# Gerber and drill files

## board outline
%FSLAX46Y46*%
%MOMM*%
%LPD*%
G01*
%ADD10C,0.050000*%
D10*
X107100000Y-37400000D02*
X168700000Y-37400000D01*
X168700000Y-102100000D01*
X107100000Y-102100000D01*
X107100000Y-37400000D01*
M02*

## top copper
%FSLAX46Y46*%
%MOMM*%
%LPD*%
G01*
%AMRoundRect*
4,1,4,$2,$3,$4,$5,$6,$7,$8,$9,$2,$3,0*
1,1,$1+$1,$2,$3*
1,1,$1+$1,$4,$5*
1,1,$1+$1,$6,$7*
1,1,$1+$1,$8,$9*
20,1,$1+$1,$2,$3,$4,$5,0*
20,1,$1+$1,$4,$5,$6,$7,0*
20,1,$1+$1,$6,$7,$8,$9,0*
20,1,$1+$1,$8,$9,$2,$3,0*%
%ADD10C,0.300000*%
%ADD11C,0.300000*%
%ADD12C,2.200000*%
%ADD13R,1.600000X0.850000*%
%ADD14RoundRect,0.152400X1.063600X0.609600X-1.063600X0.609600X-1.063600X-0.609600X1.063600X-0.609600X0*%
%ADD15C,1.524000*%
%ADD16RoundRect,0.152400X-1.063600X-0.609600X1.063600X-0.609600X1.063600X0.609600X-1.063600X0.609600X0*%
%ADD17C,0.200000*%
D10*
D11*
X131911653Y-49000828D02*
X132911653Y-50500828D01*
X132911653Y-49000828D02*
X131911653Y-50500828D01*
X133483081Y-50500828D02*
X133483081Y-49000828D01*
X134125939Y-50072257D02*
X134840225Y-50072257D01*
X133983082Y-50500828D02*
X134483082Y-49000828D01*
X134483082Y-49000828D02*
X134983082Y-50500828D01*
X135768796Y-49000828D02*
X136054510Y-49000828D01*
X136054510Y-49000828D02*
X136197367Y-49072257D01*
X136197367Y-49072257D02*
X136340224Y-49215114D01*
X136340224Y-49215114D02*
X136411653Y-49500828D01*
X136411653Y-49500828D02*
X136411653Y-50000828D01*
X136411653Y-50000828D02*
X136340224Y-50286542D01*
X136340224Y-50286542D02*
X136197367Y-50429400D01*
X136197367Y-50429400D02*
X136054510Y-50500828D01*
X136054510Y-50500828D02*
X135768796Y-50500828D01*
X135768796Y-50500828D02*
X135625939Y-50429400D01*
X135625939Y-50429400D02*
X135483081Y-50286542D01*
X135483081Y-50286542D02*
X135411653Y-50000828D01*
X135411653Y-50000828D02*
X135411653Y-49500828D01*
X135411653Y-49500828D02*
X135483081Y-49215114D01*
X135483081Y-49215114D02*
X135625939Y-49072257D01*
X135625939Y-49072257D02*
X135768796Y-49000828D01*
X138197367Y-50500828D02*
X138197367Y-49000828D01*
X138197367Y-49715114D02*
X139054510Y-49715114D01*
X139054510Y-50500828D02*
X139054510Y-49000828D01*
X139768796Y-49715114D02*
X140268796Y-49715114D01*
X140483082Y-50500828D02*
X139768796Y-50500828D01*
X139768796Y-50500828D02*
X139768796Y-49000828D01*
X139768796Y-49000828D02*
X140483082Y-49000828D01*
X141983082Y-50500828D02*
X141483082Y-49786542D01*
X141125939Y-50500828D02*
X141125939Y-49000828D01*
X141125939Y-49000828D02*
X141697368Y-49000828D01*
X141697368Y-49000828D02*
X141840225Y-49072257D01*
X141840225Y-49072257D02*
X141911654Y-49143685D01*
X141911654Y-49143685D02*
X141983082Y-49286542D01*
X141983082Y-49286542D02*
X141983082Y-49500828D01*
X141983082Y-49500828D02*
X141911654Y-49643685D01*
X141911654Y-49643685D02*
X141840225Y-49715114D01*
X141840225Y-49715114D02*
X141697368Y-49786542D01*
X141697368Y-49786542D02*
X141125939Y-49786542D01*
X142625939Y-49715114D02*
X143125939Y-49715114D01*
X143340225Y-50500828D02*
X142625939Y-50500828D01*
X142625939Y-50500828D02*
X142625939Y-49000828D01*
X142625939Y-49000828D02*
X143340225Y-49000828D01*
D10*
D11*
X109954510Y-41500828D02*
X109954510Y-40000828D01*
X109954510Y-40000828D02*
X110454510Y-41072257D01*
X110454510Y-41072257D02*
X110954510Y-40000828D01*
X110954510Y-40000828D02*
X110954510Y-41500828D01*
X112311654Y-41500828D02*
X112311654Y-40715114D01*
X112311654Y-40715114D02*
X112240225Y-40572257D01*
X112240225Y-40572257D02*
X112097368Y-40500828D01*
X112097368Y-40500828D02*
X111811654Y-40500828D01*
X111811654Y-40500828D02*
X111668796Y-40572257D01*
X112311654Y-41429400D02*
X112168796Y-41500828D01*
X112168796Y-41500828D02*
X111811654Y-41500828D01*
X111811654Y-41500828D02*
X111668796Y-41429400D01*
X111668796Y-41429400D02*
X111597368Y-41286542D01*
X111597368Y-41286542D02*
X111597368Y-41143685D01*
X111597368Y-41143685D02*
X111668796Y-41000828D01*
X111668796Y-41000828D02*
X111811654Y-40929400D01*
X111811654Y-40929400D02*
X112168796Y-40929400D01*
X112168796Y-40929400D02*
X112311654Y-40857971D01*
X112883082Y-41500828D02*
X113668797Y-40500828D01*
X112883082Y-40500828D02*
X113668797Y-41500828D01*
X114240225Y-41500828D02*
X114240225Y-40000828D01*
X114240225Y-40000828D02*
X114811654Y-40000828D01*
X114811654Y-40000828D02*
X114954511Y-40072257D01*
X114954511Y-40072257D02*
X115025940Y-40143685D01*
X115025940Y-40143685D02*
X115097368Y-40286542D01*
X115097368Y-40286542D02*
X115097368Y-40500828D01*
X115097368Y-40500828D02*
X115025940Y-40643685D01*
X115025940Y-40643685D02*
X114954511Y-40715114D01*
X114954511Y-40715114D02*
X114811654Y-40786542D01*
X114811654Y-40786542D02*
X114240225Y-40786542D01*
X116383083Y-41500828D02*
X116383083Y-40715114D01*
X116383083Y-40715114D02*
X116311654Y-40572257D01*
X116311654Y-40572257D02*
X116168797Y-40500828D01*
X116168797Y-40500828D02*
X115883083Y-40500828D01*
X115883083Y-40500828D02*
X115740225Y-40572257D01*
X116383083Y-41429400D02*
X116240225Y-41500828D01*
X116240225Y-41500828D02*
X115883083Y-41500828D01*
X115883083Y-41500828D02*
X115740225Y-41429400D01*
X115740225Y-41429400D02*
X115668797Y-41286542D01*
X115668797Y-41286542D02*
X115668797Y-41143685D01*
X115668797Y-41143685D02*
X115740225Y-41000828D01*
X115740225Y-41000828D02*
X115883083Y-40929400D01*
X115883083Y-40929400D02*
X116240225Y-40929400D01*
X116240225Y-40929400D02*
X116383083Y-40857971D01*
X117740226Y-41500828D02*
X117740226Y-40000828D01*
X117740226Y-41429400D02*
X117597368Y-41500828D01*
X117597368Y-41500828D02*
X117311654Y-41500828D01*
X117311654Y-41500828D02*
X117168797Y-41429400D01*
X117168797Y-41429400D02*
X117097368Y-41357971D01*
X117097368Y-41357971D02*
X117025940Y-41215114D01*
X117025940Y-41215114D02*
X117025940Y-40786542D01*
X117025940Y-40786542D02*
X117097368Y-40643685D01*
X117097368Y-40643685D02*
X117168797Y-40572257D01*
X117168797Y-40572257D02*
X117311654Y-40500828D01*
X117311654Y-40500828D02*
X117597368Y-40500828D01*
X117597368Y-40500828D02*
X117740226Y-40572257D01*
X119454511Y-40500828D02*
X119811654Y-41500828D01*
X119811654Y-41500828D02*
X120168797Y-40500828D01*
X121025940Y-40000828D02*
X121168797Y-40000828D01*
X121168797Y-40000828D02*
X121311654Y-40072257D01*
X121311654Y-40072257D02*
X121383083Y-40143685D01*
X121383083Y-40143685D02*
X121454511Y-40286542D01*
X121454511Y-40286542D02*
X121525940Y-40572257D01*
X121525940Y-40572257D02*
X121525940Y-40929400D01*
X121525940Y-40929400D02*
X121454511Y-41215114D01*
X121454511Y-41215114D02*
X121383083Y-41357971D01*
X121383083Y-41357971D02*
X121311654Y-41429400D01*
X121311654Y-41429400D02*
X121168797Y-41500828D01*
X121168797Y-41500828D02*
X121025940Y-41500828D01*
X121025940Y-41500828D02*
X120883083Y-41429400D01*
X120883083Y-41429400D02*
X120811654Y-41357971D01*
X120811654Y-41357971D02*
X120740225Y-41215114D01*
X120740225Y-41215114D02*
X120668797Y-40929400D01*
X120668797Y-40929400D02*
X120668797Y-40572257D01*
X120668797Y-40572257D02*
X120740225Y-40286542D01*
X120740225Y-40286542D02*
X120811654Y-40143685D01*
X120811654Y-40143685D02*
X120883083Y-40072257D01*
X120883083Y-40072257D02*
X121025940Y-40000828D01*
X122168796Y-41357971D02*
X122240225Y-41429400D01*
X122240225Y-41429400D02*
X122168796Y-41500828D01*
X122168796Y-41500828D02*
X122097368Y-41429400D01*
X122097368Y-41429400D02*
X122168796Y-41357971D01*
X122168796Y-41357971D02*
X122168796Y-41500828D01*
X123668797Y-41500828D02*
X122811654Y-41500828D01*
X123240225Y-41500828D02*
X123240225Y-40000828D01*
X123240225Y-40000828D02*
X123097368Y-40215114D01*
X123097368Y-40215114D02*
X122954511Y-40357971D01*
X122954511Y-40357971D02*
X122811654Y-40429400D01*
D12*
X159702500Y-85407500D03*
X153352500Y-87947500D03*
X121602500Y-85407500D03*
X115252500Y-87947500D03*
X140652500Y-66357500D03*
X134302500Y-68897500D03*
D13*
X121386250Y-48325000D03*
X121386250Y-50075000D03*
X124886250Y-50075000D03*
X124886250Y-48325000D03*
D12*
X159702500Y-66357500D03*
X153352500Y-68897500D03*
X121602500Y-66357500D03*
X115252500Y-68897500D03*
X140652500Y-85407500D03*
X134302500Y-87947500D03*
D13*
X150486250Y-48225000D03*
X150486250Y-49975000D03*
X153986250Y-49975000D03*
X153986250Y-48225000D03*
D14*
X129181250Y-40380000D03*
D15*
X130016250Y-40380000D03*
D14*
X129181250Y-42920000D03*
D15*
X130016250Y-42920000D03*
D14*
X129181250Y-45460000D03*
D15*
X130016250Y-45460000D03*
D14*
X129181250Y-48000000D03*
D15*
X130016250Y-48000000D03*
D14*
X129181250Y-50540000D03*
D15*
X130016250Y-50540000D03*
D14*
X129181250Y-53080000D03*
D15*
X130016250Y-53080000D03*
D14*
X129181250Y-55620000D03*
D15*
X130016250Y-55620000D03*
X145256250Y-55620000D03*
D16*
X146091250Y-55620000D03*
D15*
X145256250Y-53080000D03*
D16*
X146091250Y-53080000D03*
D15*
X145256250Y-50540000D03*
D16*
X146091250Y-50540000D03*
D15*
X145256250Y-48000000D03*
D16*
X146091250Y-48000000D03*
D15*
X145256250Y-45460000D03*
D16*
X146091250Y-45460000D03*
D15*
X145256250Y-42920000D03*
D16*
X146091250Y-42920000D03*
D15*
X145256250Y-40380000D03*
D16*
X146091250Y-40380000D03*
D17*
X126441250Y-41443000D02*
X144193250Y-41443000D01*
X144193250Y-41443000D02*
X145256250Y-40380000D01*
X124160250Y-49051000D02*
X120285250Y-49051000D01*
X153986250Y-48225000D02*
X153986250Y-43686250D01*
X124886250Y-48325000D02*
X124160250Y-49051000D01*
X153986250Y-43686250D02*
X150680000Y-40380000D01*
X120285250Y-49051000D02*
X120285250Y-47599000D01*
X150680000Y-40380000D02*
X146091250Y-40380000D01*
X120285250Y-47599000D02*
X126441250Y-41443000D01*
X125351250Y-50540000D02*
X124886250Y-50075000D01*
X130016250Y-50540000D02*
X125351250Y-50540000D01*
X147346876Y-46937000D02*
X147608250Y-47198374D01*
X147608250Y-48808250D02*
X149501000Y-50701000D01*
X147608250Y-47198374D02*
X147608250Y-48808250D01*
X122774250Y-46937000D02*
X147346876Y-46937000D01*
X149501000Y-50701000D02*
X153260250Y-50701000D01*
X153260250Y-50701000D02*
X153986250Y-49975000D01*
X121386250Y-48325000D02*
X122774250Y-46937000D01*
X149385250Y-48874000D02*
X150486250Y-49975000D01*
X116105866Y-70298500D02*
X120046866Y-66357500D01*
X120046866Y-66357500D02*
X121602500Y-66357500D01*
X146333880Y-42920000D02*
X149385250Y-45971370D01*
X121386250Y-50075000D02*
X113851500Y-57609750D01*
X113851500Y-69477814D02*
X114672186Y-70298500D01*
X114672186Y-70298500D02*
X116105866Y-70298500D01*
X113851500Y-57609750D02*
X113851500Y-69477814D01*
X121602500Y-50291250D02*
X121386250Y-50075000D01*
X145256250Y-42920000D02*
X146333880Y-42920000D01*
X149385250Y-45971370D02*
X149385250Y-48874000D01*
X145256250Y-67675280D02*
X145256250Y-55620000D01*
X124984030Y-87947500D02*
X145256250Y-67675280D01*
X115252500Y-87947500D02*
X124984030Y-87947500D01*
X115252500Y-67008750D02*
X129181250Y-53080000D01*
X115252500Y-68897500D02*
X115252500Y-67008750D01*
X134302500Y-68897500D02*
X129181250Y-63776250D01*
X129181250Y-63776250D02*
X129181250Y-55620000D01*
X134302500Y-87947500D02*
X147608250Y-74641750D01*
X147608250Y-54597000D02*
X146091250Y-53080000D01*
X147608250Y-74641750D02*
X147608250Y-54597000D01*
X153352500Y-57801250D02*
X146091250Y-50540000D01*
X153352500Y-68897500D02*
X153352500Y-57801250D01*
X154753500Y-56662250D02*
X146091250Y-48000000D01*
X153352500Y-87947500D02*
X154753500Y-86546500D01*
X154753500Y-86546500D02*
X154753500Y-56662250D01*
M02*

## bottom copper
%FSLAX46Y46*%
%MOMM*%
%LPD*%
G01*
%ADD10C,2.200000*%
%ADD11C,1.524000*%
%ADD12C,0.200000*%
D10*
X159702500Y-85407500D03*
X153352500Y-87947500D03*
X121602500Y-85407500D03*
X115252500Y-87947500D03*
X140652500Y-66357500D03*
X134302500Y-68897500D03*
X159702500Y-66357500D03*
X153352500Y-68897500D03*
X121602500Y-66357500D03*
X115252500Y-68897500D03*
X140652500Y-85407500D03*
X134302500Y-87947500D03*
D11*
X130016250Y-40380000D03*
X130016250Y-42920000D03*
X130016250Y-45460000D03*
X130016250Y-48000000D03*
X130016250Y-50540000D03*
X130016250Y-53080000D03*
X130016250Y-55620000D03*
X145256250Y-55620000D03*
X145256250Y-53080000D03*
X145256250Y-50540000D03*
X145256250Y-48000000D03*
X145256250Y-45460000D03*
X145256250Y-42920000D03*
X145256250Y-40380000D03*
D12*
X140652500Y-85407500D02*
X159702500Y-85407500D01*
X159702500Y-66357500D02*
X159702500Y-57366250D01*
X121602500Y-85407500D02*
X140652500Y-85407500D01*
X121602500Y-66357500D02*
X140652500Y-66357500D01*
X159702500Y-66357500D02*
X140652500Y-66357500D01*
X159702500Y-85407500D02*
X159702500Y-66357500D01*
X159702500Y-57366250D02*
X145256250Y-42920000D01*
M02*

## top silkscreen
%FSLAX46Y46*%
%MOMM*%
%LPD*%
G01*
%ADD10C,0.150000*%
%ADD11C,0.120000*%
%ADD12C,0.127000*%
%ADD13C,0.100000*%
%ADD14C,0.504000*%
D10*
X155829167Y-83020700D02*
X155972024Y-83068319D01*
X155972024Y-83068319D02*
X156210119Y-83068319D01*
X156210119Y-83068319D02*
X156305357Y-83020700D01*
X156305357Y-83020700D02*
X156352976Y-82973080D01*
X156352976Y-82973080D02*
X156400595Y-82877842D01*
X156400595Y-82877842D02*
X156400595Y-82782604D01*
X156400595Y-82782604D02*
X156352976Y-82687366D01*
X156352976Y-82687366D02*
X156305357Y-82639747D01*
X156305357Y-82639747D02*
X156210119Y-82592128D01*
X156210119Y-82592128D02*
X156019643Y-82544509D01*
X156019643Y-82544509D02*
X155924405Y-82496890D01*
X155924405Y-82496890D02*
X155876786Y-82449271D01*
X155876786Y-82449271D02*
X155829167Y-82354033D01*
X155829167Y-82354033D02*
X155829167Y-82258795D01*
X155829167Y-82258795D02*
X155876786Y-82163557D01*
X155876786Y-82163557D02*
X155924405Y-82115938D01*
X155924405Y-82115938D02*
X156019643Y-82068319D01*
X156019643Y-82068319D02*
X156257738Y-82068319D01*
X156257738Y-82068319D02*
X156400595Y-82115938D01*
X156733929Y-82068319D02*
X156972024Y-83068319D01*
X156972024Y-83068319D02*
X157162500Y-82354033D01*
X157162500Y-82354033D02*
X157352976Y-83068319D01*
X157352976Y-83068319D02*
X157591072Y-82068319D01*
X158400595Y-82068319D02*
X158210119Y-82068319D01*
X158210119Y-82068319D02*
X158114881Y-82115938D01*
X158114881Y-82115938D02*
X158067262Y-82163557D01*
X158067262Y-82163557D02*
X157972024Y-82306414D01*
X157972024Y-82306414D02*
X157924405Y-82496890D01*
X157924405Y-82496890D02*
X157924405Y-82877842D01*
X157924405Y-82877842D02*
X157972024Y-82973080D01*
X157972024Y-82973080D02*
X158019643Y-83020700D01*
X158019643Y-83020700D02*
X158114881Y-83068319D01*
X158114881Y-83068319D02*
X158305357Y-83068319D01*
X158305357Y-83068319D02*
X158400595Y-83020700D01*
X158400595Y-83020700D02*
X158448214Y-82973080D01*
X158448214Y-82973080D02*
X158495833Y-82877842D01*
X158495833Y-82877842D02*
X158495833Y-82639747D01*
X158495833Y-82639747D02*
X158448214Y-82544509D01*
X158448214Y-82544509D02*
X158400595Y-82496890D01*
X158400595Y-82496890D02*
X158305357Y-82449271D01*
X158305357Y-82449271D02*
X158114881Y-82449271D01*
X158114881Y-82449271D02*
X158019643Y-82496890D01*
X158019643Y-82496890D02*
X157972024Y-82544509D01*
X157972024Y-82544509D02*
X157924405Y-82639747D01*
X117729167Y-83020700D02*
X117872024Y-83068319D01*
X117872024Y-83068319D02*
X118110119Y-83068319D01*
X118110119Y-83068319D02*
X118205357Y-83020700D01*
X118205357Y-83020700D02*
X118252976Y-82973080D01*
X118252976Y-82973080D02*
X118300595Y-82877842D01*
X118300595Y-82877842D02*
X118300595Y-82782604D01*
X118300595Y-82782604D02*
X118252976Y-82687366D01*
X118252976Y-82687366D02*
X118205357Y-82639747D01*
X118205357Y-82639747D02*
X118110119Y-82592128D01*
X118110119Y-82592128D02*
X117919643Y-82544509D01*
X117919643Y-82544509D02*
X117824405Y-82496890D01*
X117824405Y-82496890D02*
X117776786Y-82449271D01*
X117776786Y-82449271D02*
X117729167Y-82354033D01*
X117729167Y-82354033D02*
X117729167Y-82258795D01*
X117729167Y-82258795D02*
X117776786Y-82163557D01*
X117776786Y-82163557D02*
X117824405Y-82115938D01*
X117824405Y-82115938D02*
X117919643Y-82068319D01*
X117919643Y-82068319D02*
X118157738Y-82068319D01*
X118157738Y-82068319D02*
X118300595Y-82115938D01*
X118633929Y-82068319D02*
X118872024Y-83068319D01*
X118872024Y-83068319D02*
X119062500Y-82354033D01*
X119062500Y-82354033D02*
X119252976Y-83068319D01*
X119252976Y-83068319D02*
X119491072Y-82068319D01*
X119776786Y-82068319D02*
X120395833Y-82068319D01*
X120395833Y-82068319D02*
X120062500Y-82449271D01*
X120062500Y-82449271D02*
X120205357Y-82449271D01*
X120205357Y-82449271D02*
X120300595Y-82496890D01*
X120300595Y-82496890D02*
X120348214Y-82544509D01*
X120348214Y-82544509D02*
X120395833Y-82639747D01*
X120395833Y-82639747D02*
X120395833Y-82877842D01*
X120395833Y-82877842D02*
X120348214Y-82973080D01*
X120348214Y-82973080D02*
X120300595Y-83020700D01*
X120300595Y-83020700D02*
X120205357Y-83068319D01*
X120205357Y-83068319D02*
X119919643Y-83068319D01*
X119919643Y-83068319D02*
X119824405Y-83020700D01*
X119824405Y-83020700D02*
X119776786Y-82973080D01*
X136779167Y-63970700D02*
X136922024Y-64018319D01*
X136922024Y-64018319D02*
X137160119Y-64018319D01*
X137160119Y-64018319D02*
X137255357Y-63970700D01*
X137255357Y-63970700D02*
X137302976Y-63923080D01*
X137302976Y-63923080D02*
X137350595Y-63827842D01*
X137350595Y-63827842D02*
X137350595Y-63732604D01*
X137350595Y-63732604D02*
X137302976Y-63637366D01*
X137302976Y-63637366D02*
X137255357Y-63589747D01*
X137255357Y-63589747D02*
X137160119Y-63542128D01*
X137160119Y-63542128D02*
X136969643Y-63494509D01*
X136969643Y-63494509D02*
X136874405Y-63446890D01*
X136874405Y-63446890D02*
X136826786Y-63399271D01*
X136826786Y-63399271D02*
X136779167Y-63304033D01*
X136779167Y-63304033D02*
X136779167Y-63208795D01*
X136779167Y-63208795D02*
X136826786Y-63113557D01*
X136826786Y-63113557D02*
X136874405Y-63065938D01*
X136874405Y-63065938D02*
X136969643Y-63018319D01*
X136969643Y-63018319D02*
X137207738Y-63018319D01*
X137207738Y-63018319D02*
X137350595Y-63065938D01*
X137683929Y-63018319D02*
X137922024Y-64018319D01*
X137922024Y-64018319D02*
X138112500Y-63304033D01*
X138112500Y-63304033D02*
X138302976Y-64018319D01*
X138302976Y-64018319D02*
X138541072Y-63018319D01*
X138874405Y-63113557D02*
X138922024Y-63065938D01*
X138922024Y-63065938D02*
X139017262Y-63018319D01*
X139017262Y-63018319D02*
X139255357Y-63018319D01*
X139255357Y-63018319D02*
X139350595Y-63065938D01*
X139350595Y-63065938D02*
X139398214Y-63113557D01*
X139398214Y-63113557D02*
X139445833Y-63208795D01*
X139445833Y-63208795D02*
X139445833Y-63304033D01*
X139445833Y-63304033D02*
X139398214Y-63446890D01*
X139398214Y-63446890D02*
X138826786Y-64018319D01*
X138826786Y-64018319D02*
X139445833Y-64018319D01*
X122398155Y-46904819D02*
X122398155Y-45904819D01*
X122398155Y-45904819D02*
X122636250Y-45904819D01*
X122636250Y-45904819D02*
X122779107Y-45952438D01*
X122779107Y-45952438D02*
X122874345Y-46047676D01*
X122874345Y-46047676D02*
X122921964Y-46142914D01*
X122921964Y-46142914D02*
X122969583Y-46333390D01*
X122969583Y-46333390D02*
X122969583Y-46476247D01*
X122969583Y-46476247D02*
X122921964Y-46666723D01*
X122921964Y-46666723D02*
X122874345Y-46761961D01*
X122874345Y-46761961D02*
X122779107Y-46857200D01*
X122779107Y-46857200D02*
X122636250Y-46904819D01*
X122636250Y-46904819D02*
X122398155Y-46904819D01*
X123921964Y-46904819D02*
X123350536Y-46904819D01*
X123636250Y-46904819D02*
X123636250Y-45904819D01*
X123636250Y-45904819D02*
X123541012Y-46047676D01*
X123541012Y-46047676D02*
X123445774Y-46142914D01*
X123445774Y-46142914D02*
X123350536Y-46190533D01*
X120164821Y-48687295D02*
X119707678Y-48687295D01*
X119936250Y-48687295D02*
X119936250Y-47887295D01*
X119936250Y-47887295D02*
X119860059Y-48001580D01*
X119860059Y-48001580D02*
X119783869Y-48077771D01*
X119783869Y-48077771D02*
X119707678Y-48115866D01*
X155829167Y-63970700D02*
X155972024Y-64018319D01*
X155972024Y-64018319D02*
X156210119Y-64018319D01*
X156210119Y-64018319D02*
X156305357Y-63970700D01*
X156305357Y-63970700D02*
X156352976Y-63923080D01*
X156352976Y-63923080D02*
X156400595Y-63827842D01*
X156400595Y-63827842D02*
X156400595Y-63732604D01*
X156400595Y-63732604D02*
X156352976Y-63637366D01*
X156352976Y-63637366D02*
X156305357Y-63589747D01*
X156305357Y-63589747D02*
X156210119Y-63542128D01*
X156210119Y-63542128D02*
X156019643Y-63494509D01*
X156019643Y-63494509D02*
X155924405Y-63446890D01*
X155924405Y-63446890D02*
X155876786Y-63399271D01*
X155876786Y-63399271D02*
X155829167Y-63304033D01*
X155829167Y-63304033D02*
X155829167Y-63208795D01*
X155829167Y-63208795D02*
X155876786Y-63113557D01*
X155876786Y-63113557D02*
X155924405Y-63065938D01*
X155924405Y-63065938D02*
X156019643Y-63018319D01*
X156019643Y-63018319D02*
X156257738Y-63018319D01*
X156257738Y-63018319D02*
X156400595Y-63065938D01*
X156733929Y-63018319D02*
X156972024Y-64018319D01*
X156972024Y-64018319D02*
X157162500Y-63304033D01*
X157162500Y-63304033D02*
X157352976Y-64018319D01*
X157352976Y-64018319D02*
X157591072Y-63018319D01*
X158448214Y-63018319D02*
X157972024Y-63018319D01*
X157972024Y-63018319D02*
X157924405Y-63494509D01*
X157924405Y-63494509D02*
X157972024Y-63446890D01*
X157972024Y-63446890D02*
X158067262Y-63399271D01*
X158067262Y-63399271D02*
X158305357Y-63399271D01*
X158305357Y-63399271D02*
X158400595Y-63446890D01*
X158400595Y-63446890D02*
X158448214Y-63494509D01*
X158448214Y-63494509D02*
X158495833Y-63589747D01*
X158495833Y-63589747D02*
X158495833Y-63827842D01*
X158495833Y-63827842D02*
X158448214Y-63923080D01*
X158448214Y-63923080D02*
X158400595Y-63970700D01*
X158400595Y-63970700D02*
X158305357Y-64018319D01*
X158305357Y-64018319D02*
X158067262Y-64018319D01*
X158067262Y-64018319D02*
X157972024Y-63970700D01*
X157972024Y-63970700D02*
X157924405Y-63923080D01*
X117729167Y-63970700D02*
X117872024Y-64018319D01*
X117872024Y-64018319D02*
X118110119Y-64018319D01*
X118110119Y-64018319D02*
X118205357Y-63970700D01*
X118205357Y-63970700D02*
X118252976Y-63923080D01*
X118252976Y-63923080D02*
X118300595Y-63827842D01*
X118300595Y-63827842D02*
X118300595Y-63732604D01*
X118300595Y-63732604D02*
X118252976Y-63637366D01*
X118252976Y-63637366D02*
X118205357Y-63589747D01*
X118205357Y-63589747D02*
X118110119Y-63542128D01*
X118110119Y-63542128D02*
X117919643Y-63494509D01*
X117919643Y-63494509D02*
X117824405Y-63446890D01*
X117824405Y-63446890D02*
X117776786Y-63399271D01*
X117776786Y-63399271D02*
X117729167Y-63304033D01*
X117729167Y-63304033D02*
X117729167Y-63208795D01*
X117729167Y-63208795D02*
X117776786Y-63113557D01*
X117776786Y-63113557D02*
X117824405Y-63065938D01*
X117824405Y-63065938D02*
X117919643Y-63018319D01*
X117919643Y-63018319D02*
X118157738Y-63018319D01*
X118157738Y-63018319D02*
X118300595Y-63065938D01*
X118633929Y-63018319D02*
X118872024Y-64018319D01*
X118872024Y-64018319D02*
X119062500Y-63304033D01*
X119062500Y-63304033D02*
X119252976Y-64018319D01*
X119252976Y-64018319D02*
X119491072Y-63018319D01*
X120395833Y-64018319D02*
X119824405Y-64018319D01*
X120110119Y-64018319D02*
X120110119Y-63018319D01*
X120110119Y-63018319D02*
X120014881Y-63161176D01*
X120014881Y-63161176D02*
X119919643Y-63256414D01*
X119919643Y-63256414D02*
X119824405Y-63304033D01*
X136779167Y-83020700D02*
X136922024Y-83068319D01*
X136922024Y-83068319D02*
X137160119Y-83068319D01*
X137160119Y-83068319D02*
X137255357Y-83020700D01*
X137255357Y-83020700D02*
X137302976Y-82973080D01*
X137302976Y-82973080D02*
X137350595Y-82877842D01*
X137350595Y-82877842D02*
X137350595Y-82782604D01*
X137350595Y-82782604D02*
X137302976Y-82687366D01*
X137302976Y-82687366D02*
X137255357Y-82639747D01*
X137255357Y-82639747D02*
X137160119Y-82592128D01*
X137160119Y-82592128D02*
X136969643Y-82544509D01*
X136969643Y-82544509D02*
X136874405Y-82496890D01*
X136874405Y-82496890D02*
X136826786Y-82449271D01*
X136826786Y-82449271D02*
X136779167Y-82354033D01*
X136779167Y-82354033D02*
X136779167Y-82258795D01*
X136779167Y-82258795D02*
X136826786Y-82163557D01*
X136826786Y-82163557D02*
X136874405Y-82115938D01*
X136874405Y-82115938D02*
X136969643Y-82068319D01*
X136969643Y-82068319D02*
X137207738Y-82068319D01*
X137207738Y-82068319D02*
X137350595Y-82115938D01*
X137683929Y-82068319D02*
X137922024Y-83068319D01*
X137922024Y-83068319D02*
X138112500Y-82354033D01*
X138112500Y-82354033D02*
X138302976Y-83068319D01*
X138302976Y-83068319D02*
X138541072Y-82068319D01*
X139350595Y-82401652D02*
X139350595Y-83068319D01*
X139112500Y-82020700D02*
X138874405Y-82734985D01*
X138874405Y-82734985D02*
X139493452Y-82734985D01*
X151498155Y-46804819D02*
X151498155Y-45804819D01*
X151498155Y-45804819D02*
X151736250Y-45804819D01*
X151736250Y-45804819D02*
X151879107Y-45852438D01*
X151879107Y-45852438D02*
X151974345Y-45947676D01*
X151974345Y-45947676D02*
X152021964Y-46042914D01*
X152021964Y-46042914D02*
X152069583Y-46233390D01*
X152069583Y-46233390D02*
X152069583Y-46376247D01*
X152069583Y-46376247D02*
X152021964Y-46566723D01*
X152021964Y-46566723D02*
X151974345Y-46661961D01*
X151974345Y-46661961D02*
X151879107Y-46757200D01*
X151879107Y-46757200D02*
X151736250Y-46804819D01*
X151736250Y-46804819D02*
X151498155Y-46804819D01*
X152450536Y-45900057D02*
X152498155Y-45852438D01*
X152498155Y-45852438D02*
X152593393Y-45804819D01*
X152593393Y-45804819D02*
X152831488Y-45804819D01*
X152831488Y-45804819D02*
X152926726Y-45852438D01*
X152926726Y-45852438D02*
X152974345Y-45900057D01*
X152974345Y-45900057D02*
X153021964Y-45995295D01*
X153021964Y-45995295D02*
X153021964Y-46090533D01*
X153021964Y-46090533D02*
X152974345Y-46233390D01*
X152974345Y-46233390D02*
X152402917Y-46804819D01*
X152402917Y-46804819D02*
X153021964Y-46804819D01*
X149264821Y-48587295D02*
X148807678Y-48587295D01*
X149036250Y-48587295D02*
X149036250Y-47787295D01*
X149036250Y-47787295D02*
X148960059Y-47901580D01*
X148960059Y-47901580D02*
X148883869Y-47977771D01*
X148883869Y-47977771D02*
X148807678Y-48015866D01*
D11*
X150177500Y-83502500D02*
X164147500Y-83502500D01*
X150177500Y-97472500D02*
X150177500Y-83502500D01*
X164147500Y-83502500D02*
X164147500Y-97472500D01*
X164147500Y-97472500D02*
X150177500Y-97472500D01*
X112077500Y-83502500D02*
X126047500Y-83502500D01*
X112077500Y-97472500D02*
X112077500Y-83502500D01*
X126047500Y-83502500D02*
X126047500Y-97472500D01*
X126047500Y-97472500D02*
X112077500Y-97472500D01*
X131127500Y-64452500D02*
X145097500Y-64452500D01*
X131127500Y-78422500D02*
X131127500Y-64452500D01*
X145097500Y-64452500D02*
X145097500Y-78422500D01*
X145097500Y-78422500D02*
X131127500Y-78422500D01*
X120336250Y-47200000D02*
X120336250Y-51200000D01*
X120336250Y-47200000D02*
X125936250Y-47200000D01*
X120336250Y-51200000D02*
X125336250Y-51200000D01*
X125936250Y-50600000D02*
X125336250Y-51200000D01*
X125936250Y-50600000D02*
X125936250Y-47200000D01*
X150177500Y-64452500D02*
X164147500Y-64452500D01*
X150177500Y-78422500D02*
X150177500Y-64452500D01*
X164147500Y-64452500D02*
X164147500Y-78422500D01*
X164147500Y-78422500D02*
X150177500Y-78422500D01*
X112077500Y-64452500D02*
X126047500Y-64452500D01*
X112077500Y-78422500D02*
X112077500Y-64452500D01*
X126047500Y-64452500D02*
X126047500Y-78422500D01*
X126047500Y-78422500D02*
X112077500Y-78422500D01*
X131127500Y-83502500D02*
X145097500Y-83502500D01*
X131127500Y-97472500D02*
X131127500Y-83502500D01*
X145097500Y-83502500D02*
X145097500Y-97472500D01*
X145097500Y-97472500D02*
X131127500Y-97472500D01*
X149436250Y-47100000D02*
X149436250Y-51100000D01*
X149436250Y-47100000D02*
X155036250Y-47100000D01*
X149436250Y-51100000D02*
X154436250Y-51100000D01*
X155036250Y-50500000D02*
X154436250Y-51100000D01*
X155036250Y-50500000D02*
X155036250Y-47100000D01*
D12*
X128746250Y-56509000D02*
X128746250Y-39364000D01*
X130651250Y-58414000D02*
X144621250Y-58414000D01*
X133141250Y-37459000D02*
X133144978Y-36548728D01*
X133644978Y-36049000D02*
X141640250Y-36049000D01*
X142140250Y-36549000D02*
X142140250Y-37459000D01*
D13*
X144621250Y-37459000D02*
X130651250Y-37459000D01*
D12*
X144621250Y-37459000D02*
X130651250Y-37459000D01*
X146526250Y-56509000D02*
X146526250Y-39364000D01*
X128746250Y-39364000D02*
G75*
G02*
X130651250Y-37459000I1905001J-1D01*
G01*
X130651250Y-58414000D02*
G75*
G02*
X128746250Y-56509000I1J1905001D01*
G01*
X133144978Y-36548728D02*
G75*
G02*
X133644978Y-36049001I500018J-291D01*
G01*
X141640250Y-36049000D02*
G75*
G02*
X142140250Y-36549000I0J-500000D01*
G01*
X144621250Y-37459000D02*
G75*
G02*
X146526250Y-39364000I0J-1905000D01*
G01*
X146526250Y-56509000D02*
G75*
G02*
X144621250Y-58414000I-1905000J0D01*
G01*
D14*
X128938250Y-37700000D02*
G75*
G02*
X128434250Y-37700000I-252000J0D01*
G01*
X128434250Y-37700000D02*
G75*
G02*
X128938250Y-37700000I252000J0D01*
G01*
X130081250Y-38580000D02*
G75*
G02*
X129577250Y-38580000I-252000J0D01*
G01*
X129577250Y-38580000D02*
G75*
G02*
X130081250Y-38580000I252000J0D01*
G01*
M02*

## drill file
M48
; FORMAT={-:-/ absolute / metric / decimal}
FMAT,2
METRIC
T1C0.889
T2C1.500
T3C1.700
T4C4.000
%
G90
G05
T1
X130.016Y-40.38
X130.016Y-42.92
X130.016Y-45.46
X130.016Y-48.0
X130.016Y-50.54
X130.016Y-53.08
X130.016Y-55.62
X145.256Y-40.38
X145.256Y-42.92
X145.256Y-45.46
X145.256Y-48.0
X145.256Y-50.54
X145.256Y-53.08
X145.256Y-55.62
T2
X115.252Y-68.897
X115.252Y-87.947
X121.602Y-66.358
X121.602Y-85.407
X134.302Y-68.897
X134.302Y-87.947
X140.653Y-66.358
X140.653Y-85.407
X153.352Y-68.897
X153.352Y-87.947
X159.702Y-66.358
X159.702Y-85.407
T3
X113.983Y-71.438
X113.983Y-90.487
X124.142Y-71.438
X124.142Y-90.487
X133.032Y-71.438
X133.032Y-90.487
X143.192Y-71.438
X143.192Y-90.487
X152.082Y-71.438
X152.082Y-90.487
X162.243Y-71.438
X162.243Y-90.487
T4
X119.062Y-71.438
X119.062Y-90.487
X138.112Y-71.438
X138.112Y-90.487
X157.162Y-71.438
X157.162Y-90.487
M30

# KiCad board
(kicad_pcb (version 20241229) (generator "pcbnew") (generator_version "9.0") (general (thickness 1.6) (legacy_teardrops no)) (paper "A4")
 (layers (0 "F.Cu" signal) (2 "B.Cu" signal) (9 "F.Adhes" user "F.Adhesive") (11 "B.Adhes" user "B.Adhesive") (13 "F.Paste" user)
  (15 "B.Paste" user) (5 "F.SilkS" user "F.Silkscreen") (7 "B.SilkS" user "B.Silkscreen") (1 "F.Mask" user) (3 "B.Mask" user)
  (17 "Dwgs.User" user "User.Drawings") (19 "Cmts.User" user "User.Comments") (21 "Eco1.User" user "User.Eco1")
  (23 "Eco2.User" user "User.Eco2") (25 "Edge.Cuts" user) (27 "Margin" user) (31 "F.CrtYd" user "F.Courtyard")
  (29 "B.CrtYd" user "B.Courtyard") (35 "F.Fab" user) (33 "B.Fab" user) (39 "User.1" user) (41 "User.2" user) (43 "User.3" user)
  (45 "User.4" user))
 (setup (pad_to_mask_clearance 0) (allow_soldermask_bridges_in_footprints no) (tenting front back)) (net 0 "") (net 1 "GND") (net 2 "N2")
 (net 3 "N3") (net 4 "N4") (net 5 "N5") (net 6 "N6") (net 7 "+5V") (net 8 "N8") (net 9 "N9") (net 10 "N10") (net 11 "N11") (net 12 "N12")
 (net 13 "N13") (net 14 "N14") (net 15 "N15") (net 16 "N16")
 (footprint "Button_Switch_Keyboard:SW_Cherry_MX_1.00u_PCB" (layer "F.Cu") (at 159.7025 85.4075)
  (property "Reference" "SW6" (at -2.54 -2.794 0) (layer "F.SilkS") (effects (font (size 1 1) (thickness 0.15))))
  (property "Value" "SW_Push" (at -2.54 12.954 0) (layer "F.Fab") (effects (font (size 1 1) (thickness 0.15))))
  (fp_line (start -9.525 -1.905) (end 4.445 -1.905) (stroke (width 0.12) (type solid)) (layer "F.SilkS"))
  (fp_line (start -9.525 12.065) (end -9.525 -1.905) (stroke (width 0.12) (type solid)) (layer "F.SilkS"))
  (fp_line (start 4.445 -1.905) (end 4.445 12.065) (stroke (width 0.12) (type solid)) (layer "F.SilkS"))
  (fp_line (start 4.445 12.065) (end -9.525 12.065) (stroke (width 0.12) (type solid)) (layer "F.SilkS"))
  (pad "" np_thru_hole circle (at -7.62 5.08) (size 1.7 1.7) (drill 1.7) (layers "*.Cu" "*.Mask"))
  (pad "" np_thru_hole circle (at -2.54 5.08) (size 4 4) (drill 4) (layers "*.Cu" "*.Mask"))
  (pad "" np_thru_hole circle (at 2.54 5.08) (size 1.7 1.7) (drill 1.7) (layers "*.Cu" "*.Mask"))
  (pad "1" thru_hole circle (at 0 0) (size 2.2 2.2) (drill 1.5) (layers "*.Cu" "*.Mask") (remove_unused_layers no) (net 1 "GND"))
  (pad "2" thru_hole circle (at -6.35 2.54) (size 2.2 2.2) (drill 1.5) (layers "*.Cu" "*.Mask") (remove_unused_layers no) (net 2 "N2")))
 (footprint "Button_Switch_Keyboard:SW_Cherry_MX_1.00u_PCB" (layer "F.Cu") (at 121.6025 85.4075)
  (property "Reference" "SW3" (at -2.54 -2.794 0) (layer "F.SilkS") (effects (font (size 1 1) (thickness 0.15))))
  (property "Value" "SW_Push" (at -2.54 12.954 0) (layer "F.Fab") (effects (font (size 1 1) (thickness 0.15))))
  (fp_line (start -9.525 -1.905) (end 4.445 -1.905) (stroke (width 0.12) (type solid)) (layer "F.SilkS"))
  (fp_line (start -9.525 12.065) (end -9.525 -1.905) (stroke (width 0.12) (type solid)) (layer "F.SilkS"))
  (fp_line (start 4.445 -1.905) (end 4.445 12.065) (stroke (width 0.12) (type solid)) (layer "F.SilkS"))
  (fp_line (start 4.445 12.065) (end -9.525 12.065) (stroke (width 0.12) (type solid)) (layer "F.SilkS"))
  (pad "" np_thru_hole circle (at -7.62 5.08) (size 1.7 1.7) (drill 1.7) (layers "*.Cu" "*.Mask"))
  (pad "" np_thru_hole circle (at -2.54 5.08) (size 4 4) (drill 4) (layers "*.Cu" "*.Mask"))
  (pad "" np_thru_hole circle (at 2.54 5.08) (size 1.7 1.7) (drill 1.7) (layers "*.Cu" "*.Mask"))
  (pad "1" thru_hole circle (at 0 0) (size 2.2 2.2) (drill 1.5) (layers "*.Cu" "*.Mask") (remove_unused_layers no) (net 1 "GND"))
  (pad "2" thru_hole circle (at -6.35 2.54) (size 2.2 2.2) (drill 1.5) (layers "*.Cu" "*.Mask") (remove_unused_layers no) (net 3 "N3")))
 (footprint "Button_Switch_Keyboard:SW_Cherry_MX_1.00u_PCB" (layer "F.Cu") (at 140.6525 66.3575)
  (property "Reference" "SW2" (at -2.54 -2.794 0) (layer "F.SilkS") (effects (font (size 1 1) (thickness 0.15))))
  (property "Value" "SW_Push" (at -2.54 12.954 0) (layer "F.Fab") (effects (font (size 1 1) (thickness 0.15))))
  (fp_line (start -9.525 -1.905) (end 4.445 -1.905) (stroke (width 0.12) (type solid)) (layer "F.SilkS"))
  (fp_line (start -9.525 12.065) (end -9.525 -1.905) (stroke (width 0.12) (type solid)) (layer "F.SilkS"))
  (fp_line (start 4.445 -1.905) (end 4.445 12.065) (stroke (width 0.12) (type solid)) (layer "F.SilkS"))
  (fp_line (start 4.445 12.065) (end -9.525 12.065) (stroke (width 0.12) (type solid)) (layer "F.SilkS"))
  (pad "" np_thru_hole circle (at -7.62 5.08) (size 1.7 1.7) (drill 1.7) (layers "*.Cu" "*.Mask"))
  (pad "" np_thru_hole circle (at -2.54 5.08) (size 4 4) (drill 4) (layers "*.Cu" "*.Mask"))
  (pad "" np_thru_hole circle (at 2.54 5.08) (size 1.7 1.7) (drill 1.7) (layers "*.Cu" "*.Mask"))
  (pad "1" thru_hole circle (at 0 0) (size 2.2 2.2) (drill 1.5) (layers "*.Cu" "*.Mask") (remove_unused_layers no) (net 1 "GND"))
  (pad "2" thru_hole circle (at -6.35 2.54) (size 2.2 2.2) (drill 1.5) (layers "*.Cu" "*.Mask") (remove_unused_layers no) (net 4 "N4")))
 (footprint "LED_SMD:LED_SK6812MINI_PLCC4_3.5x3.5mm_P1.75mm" (layer "F.Cu") (at 123.13625 49.2)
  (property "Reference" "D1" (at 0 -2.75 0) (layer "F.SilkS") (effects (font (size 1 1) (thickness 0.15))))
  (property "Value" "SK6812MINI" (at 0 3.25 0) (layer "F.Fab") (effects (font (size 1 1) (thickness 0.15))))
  (fp_line (start -2.8 -2) (end -2.8 2) (stroke (width 0.12) (type default)) (layer "F.SilkS"))
  (fp_line (start -2.8 -2) (end 2.8 -2) (stroke (width 0.12) (type solid)) (layer "F.SilkS"))
  (fp_line (start -2.8 2) (end 2.2 2) (stroke (width 0.12) (type solid)) (layer "F.SilkS"))
  (fp_line (start 2.8 1.4) (end 2.2 2) (stroke (width 0.12) (type default)) (layer "F.SilkS"))
  (fp_line (start 2.8 1.4) (end 2.8 -2) (stroke (width 0.12) (type solid)) (layer "F.SilkS"))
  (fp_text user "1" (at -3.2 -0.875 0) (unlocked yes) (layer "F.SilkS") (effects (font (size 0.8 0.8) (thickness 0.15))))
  (pad "1" smd rect (at -1.75 -0.875) (size 1.6 0.85) (layers "F.Cu" "F.Mask" "F.Paste") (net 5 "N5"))
  (pad "2" smd rect (at -1.75 0.875) (size 1.6 0.85) (layers "F.Cu" "F.Mask" "F.Paste") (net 1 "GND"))
  (pad "3" smd rect (at 1.75 0.875) (size 1.6 0.85) (layers "F.Cu" "F.Mask" "F.Paste") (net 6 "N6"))
  (pad "4" smd rect (at 1.75 -0.875) (size 1.6 0.85) (layers "F.Cu" "F.Mask" "F.Paste") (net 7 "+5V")))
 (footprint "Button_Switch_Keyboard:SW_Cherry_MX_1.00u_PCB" (layer "F.Cu") (at 159.7025 66.3575)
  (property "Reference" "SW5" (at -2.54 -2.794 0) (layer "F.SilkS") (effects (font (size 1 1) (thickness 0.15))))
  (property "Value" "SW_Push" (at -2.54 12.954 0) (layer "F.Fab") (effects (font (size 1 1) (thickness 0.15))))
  (fp_line (start -9.525 -1.905) (end 4.445 -1.905) (stroke (width 0.12) (type solid)) (layer "F.SilkS"))
  (fp_line (start -9.525 12.065) (end -9.525 -1.905) (stroke (width 0.12) (type solid)) (layer "F.SilkS"))
  (fp_line (start 4.445 -1.905) (end 4.445 12.065) (stroke (width 0.12) (type solid)) (layer "F.SilkS"))
  (fp_line (start 4.445 12.065) (end -9.525 12.065) (stroke (width 0.12) (type solid)) (layer "F.SilkS"))
  (pad "" np_thru_hole circle (at -7.62 5.08) (size 1.7 1.7) (drill 1.7) (layers "*.Cu" "*.Mask"))
  (pad "" np_thru_hole circle (at -2.54 5.08) (size 4 4) (drill 4) (layers "*.Cu" "*.Mask"))
  (pad "" np_thru_hole circle (at 2.54 5.08) (size 1.7 1.7) (drill 1.7) (layers "*.Cu" "*.Mask"))
  (pad "1" thru_hole circle (at 0 0) (size 2.2 2.2) (drill 1.5) (layers "*.Cu" "*.Mask") (remove_unused_layers no) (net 1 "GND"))
  (pad "2" thru_hole circle (at -6.35 2.54) (size 2.2 2.2) (drill 1.5) (layers "*.Cu" "*.Mask") (remove_unused_layers no) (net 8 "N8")))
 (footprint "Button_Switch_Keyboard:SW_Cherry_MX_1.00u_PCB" (layer "F.Cu") (at 121.6025 66.3575)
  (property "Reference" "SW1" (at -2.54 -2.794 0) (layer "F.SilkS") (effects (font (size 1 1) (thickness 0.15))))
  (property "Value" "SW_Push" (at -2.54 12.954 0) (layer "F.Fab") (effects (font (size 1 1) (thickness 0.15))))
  (fp_line (start -9.525 -1.905) (end 4.445 -1.905) (stroke (width 0.12) (type solid)) (layer "F.SilkS"))
  (fp_line (start -9.525 12.065) (end -9.525 -1.905) (stroke (width 0.12) (type solid)) (layer "F.SilkS"))
  (fp_line (start 4.445 -1.905) (end 4.445 12.065) (stroke (width 0.12) (type solid)) (layer "F.SilkS"))
  (fp_line (start 4.445 12.065) (end -9.525 12.065) (stroke (width 0.12) (type solid)) (layer "F.SilkS"))
  (pad "" np_thru_hole circle (at -7.62 5.08) (size 1.7 1.7) (drill 1.7) (layers "*.Cu" "*.Mask"))
  (pad "" np_thru_hole circle (at -2.54 5.08) (size 4 4) (drill 4) (layers "*.Cu" "*.Mask"))
  (pad "" np_thru_hole circle (at 2.54 5.08) (size 1.7 1.7) (drill 1.7) (layers "*.Cu" "*.Mask"))
  (pad "1" thru_hole circle (at 0 0) (size 2.2 2.2) (drill 1.5) (layers "*.Cu" "*.Mask") (remove_unused_layers no) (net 1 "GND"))
  (pad "2" thru_hole circle (at -6.35 2.54) (size 2.2 2.2) (drill 1.5) (layers "*.Cu" "*.Mask") (remove_unused_layers no) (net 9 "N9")))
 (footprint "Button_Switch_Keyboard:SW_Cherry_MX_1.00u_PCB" (layer "F.Cu") (at 140.6525 85.4075)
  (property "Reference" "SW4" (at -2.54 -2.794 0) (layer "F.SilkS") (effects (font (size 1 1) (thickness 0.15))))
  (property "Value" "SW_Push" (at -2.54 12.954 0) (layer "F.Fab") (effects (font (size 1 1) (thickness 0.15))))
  (fp_line (start -9.525 -1.905) (end 4.445 -1.905) (stroke (width 0.12) (type solid)) (layer "F.SilkS"))
  (fp_line (start -9.525 12.065) (end -9.525 -1.905) (stroke (width 0.12) (type solid)) (layer "F.SilkS"))
  (fp_line (start 4.445 -1.905) (end 4.445 12.065) (stroke (width 0.12) (type solid)) (layer "F.SilkS"))
  (fp_line (start 4.445 12.065) (end -9.525 12.065) (stroke (width 0.12) (type solid)) (layer "F.SilkS"))
  (pad "" np_thru_hole circle (at -7.62 5.08) (size 1.7 1.7) (drill 1.7) (layers "*.Cu" "*.Mask"))
  (pad "" np_thru_hole circle (at -2.54 5.08) (size 4 4) (drill 4) (layers "*.Cu" "*.Mask"))
  (pad "" np_thru_hole circle (at 2.54 5.08) (size 1.7 1.7) (drill 1.7) (layers "*.Cu" "*.Mask"))
  (pad "1" thru_hole circle (at 0 0) (size 2.2 2.2) (drill 1.5) (layers "*.Cu" "*.Mask") (remove_unused_layers no) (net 1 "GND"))
  (pad "2" thru_hole circle (at -6.35 2.54) (size 2.2 2.2) (drill 1.5) (layers "*.Cu" "*.Mask") (remove_unused_layers no) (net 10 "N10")))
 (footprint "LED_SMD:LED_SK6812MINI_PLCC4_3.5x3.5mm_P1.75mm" (layer "F.Cu") (at 152.23625 49.1)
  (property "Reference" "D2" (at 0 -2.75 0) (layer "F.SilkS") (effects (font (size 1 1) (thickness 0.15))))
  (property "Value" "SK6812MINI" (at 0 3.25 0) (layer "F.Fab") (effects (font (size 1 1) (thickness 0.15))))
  (fp_line (start -2.8 -2) (end -2.8 2) (stroke (width 0.12) (type default)) (layer "F.SilkS"))
  (fp_line (start -2.8 -2) (end 2.8 -2) (stroke (width 0.12) (type solid)) (layer "F.SilkS"))
  (fp_line (start -2.8 2) (end 2.2 2) (stroke (width 0.12) (type solid)) (layer "F.SilkS"))
  (fp_line (start 2.8 1.4) (end 2.2 2) (stroke (width 0.12) (type default)) (layer "F.SilkS"))
  (fp_line (start 2.8 1.4) (end 2.8 -2) (stroke (width 0.12) (type solid)) (layer "F.SilkS"))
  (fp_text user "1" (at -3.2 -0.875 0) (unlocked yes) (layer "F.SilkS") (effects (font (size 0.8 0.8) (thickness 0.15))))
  (pad "1" smd rect (at -1.75 -0.875) (size 1.6 0.85) (layers "F.Cu" "F.Mask" "F.Paste") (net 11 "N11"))
  (pad "2" smd rect (at -1.75 0.875) (size 1.6 0.85) (layers "F.Cu" "F.Mask" "F.Paste") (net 1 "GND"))
  (pad "3" smd rect (at 1.75 0.875) (size 1.6 0.85) (layers "F.Cu" "F.Mask" "F.Paste") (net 5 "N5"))
  (pad "4" smd rect (at 1.75 -0.875) (size 1.6 0.85) (layers "F.Cu" "F.Mask" "F.Paste") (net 7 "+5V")))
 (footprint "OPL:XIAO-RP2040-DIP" (layer "F.Cu") (at 137.63625 48)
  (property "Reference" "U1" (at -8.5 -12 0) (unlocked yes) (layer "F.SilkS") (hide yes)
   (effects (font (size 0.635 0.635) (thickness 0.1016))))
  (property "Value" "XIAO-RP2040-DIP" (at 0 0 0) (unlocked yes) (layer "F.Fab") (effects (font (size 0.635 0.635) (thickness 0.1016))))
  (fp_line (start -8.89 8.509) (end -8.89 -8.636) (stroke (width 0.127) (type solid)) (layer "F.SilkS"))
  (fp_line (start -6.985 10.414) (end 6.985 10.414) (stroke (width 0.127) (type solid)) (layer "F.SilkS"))
  (fp_line (start -4.495 -10.541) (end -4.491272 -11.451272) (stroke (width 0.127) (type solid)) (layer "F.SilkS"))
  (fp_line (start -3.991272 -11.951) (end 4.004 -11.951) (stroke (width 0.127) (type solid)) (layer "F.SilkS"))
  (fp_line (start 4.504 -11.451) (end 4.504 -10.541) (stroke (width 0.127) (type solid)) (layer "F.SilkS"))
  (fp_line (start 6.985 -10.541) (end -6.985 -10.541) (stroke (width 0.1) (type solid)) (layer "F.SilkS"))
  (fp_line (start 6.985 -10.541) (end -6.985 -10.541) (stroke (width 0.127) (type solid)) (layer "F.SilkS"))
  (fp_line (start 8.89 8.509) (end 8.89 -8.636) (stroke (width 0.127) (type solid)) (layer "F.SilkS"))
  (fp_arc (start -8.89 -8.636) (mid -8.332038 -9.983038) (end -6.985 -10.541) (stroke (width 0.127) (type solid)) (layer "F.SilkS"))
  (fp_arc (start -6.985 10.414) (mid -8.332038 9.856038) (end -8.89 8.509) (stroke (width 0.127) (type solid)) (layer "F.SilkS"))
  (fp_arc (start -4.491272 -11.451272) (mid -4.344728 -11.80464) (end -3.991272 -11.951) (stroke (width 0.127) (type default))
   (layer "F.SilkS"))
  (fp_arc (start 4.004 -11.951) (mid 4.357553 -11.804553) (end 4.504 -11.451) (stroke (width 0.127) (type default)) (layer "F.SilkS"))
  (fp_arc (start 6.985 -10.541) (mid 8.332038 -9.983038) (end 8.89 -8.636) (stroke (width 0.127) (type solid)) (layer "F.SilkS"))
  (fp_arc (start 8.89 8.509) (mid 8.332038 9.856038) (end 6.985 10.414) (stroke (width 0.127) (type solid)) (layer "F.SilkS"))
  (fp_circle (center -8.95 -10.3) (end -8.95 -10.554) (stroke (width 0.5) (type solid)) (fill yes) (layer "F.SilkS"))
  (fp_circle (center -7.807 -9.42) (end -7.807 -9.674) (stroke (width 0.5) (type solid)) (fill yes) (layer "F.SilkS"))
  (pad "1" smd roundrect (at -8.455 -7.62 180) (size 2.432 1.524) (layers "F.Cu" "F.Mask") (roundrect_rratio 0.1) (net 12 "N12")
   (thermal_bridge_angle 45))
  (pad "1" thru_hole circle (at -7.62 -7.62 180) (size 1.524 1.524) (drill 0.889) (layers "*.Cu" "*.Mask") (remove_unused_layers no)
   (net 12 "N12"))
  (pad "2" smd roundrect (at -8.455 -5.08 180) (size 2.432 1.524) (layers "F.Cu" "F.Mask") (roundrect_rratio 0.1) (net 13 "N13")
   (thermal_bridge_angle 45))
  (pad "2" thru_hole circle (at -7.62 -5.08 180) (size 1.524 1.524) (drill 0.889) (layers "*.Cu" "*.Mask") (remove_unused_layers no)
   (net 13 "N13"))
  (pad "3" smd roundrect (at -8.455 -2.54 180) (size 2.432 1.524) (layers "F.Cu" "F.Mask") (roundrect_rratio 0.1) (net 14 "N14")
   (thermal_bridge_angle 45))
  (pad "3" thru_hole circle (at -7.62 -2.54 180) (size 1.524 1.524) (drill 0.889) (layers "*.Cu" "*.Mask") (remove_unused_layers no)
   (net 14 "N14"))
  (pad "4" smd roundrect (at -8.455 0 180) (size 2.432 1.524) (layers "F.Cu" "F.Mask") (roundrect_rratio 0.1) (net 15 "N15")
   (thermal_bridge_angle 45))
  (pad "4" thru_hole circle (at -7.62 0 180) (size 1.524 1.524) (drill 0.889) (layers "*.Cu" "*.Mask") (remove_unused_layers no)
   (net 15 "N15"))
  (pad "5" smd roundrect (at -8.455 2.54 180) (size 2.432 1.524) (layers "F.Cu" "F.Mask") (roundrect_rratio 0.1) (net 6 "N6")
   (thermal_bridge_angle 45))
  (pad "5" thru_hole circle (at -7.62 2.54 180) (size 1.524 1.524) (drill 0.889) (layers "*.Cu" "*.Mask") (remove_unused_layers no)
   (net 6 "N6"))
  (pad "6" smd roundrect (at -8.455 5.08 180) (size 2.432 1.524) (layers "F.Cu" "F.Mask") (roundrect_rratio 0.1) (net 9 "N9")
   (thermal_bridge_angle 45))
  (pad "6" thru_hole circle (at -7.62 5.08 180) (size 1.524 1.524) (drill 0.889) (layers "*.Cu" "*.Mask") (remove_unused_layers no)
   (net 9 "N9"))
  (pad "7" smd roundrect (at -8.455 7.62 180) (size 2.432 1.524) (layers "F.Cu" "F.Mask") (roundrect_rratio 0.1) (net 4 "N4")
   (thermal_bridge_angle 45))
  (pad "7" thru_hole circle (at -7.62 7.62 180) (size 1.524 1.524) (drill 0.889) (layers "*.Cu" "*.Mask") (remove_unused_layers no)
   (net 4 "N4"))
  (pad "8" thru_hole circle (at 7.62 7.62) (size 1.524 1.524) (drill 0.889) (layers "*.Cu" "*.Mask") (remove_unused_layers no) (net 3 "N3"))
  (pad "8" smd roundrect (at 8.455 7.62) (size 2.432 1.524) (layers "F.Cu" "F.Mask") (roundrect_rratio 0.1) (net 3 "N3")
   (thermal_bridge_angle 45))
  (pad "9" thru_hole circle (at 7.62 5.08) (size 1.524 1.524) (drill 0.889) (layers "*.Cu" "*.Mask") (remove_unused_layers no)
   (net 10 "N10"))
  (pad "9" smd roundrect (at 8.455 5.08) (size 2.432 1.524) (layers "F.Cu" "F.Mask") (roundrect_rratio 0.1) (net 10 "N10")
   (thermal_bridge_angle 45))
  (pad "10" thru_hole circle (at 7.62 2.54) (size 1.524 1.524) (drill 0.889) (layers "*.Cu" "*.Mask") (remove_unused_layers no) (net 8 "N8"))
  (pad "10" smd roundrect (at 8.455 2.54) (size 2.432 1.524) (layers "F.Cu" "F.Mask") (roundrect_rratio 0.1) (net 8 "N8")
   (thermal_bridge_angle 45))
  (pad "11" thru_hole circle (at 7.62 0) (size 1.524 1.524) (drill 0.889) (layers "*.Cu" "*.Mask") (remove_unused_layers no) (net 2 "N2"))
  (pad "11" smd roundrect (at 8.455 0) (size 2.432 1.524) (layers "F.Cu" "F.Mask") (roundrect_rratio 0.1) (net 2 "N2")
   (thermal_bridge_angle 45))
  (pad "12" thru_hole circle (at 7.62 -2.54) (size 1.524 1.524) (drill 0.889) (layers "*.Cu" "*.Mask") (remove_unused_layers no)
   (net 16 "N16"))
  (pad "12" smd roundrect (at 8.455 -2.54) (size 2.432 1.524) (layers "F.Cu" "F.Mask") (roundrect_rratio 0.1) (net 16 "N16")
   (thermal_bridge_angle 45))
  (pad "13" thru_hole circle (at 7.62 -5.08) (size 1.524 1.524) (drill 0.889) (layers "*.Cu" "*.Mask") (remove_unused_layers no)
   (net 1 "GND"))
  (pad "13" smd roundrect (at 8.455 -5.08) (size 2.432 1.524) (layers "F.Cu" "F.Mask") (roundrect_rratio 0.1) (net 1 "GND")
   (thermal_bridge_angle 45))
  (pad "14" thru_hole circle (at 7.62 -7.62) (size 1.524 1.524) (drill 0.889) (layers "*.Cu" "*.Mask") (remove_unused_layers no)
   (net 7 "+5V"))
  (pad "14" smd roundrect (at 8.455 -7.62) (size 2.432 1.524) (layers "F.Cu" "F.Mask") (roundrect_rratio 0.1) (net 7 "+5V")
   (thermal_bridge_angle 45)))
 (gr_rect (start 107.1 37.4) (end 168.7 102.1) (stroke (width 0.05) (type default)) (fill no) (layer "Edge.Cuts"))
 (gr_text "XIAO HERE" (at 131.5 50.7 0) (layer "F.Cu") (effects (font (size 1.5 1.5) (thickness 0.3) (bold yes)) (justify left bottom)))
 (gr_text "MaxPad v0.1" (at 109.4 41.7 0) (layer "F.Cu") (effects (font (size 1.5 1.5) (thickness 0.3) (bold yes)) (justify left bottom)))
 (segment (start 126.44125 41.443) (end 144.19325 41.443) (width 0.2) (layer "F.Cu") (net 7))
 (segment (start 144.19325 41.443) (end 145.25625 40.38) (width 0.2) (layer "F.Cu") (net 7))
 (segment (start 124.16025 49.051) (end 120.28525 49.051) (width 0.2) (layer "F.Cu") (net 7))
 (segment (start 153.98625 48.225) (end 153.98625 43.68625) (width 0.2) (layer "F.Cu") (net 7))
 (segment (start 124.88625 48.325) (end 124.16025 49.051) (width 0.2) (layer "F.Cu") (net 7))
 (segment (start 153.98625 43.68625) (end 150.68 40.38) (width 0.2) (layer "F.Cu") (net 7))
 (segment (start 120.28525 49.051) (end 120.28525 47.599) (width 0.2) (layer "F.Cu") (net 7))
 (segment (start 150.68 40.38) (end 146.09125 40.38) (width 0.2) (layer "F.Cu") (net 7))
 (segment (start 120.28525 47.599) (end 126.44125 41.443) (width 0.2) (layer "F.Cu") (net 7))
 (segment (start 125.35125 50.54) (end 124.88625 50.075) (width 0.2) (layer "F.Cu") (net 6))
 (segment (start 130.01625 50.54) (end 125.35125 50.54) (width 0.2) (layer "F.Cu") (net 6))
 (segment (start 147.346876 46.937) (end 147.60825 47.198374) (width 0.2) (layer "F.Cu") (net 5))
 (segment (start 147.60825 48.80825) (end 149.501 50.701) (width 0.2) (layer "F.Cu") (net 5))
 (segment (start 147.60825 47.198374) (end 147.60825 48.80825) (width 0.2) (layer "F.Cu") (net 5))
 (segment (start 122.77425 46.937) (end 147.346876 46.937) (width 0.2) (layer "F.Cu") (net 5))
 (segment (start 149.501 50.701) (end 153.26025 50.701) (width 0.2) (layer "F.Cu") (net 5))
 (segment (start 153.26025 50.701) (end 153.98625 49.975) (width 0.2) (layer "F.Cu") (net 5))
 (segment (start 121.38625 48.325) (end 122.77425 46.937) (width 0.2) (layer "F.Cu") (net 5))
 (segment (start 149.38525 48.874) (end 150.48625 49.975) (width 0.2) (layer "F.Cu") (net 1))
 (segment (start 116.105866 70.2985) (end 120.046866 66.3575) (width 0.2) (layer "F.Cu") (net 1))
 (segment (start 120.046866 66.3575) (end 121.6025 66.3575) (width 0.2) (layer "F.Cu") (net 1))
 (segment (start 146.33388 42.92) (end 149.38525 45.97137) (width 0.2) (layer "F.Cu") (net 1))
 (segment (start 121.38625 50.075) (end 113.8515 57.60975) (width 0.2) (layer "F.Cu") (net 1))
 (segment (start 113.8515 69.477814) (end 114.672186 70.2985) (width 0.2) (layer "F.Cu") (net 1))
 (segment (start 114.672186 70.2985) (end 116.105866 70.2985) (width 0.2) (layer "F.Cu") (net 1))
 (segment (start 113.8515 57.60975) (end 113.8515 69.477814) (width 0.2) (layer "F.Cu") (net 1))
 (segment (start 121.6025 50.29125) (end 121.38625 50.075) (width 0.2) (layer "F.Cu") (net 1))
 (segment (start 145.25625 42.92) (end 146.33388 42.92) (width 0.2) (layer "F.Cu") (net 1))
 (segment (start 149.38525 45.97137) (end 149.38525 48.874) (width 0.2) (layer "F.Cu") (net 1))
 (segment (start 140.6525 85.4075) (end 159.7025 85.4075) (width 0.2) (layer "B.Cu") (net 1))
 (segment (start 159.7025 66.3575) (end 159.7025 57.36625) (width 0.2) (layer "B.Cu") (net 1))
 (segment (start 121.6025 85.4075) (end 140.6525 85.4075) (width 0.2) (layer "B.Cu") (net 1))
 (segment (start 121.6025 66.3575) (end 140.6525 66.3575) (width 0.2) (layer "B.Cu") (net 1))
 (segment (start 159.7025 66.3575) (end 140.6525 66.3575) (width 0.2) (layer "B.Cu") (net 1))
 (segment (start 159.7025 85.4075) (end 159.7025 66.3575) (width 0.2) (layer "B.Cu") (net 1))
 (segment (start 159.7025 57.36625) (end 145.25625 42.92) (width 0.2) (layer "B.Cu") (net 1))
 (segment (start 145.25625 67.67528) (end 145.25625 55.62) (width 0.2) (layer "F.Cu") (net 3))
 (segment (start 124.98403 87.9475) (end 145.25625 67.67528) (width 0.2) (layer "F.Cu") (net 3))
 (segment (start 115.2525 87.9475) (end 124.98403 87.9475) (width 0.2) (layer "F.Cu") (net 3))
 (segment (start 115.2525 67.00875) (end 129.18125 53.08) (width 0.2) (layer "F.Cu") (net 9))
 (segment (start 115.2525 68.8975) (end 115.2525 67.00875) (width 0.2) (layer "F.Cu") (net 9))
 (segment (start 134.3025 68.8975) (end 129.18125 63.77625) (width 0.2) (layer "F.Cu") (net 4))
 (segment (start 129.18125 63.77625) (end 129.18125 55.62) (width 0.2) (layer "F.Cu") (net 4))
 (segment (start 134.3025 87.9475) (end 147.60825 74.64175) (width 0.2) (layer "F.Cu") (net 10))
 (segment (start 147.60825 54.597) (end 146.09125 53.08) (width 0.2) (layer "F.Cu") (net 10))
 (segment (start 147.60825 74.64175) (end 147.60825 54.597) (width 0.2) (layer "F.Cu") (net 10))
 (segment (start 153.3525 57.80125) (end 146.09125 50.54) (width 0.2) (layer "F.Cu") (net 8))
 (segment (start 153.3525 68.8975) (end 153.3525 57.80125) (width 0.2) (layer "F.Cu") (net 8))
 (segment (start 154.7535 56.66225) (end 146.09125 48) (width 0.2) (layer "F.Cu") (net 2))
 (segment (start 153.3525 87.9475) (end 154.7535 86.5465) (width 0.2) (layer "F.Cu") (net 2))
 (segment (start 154.7535 86.5465) (end 154.7535 56.66225) (width 0.2) (layer "F.Cu") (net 2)))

